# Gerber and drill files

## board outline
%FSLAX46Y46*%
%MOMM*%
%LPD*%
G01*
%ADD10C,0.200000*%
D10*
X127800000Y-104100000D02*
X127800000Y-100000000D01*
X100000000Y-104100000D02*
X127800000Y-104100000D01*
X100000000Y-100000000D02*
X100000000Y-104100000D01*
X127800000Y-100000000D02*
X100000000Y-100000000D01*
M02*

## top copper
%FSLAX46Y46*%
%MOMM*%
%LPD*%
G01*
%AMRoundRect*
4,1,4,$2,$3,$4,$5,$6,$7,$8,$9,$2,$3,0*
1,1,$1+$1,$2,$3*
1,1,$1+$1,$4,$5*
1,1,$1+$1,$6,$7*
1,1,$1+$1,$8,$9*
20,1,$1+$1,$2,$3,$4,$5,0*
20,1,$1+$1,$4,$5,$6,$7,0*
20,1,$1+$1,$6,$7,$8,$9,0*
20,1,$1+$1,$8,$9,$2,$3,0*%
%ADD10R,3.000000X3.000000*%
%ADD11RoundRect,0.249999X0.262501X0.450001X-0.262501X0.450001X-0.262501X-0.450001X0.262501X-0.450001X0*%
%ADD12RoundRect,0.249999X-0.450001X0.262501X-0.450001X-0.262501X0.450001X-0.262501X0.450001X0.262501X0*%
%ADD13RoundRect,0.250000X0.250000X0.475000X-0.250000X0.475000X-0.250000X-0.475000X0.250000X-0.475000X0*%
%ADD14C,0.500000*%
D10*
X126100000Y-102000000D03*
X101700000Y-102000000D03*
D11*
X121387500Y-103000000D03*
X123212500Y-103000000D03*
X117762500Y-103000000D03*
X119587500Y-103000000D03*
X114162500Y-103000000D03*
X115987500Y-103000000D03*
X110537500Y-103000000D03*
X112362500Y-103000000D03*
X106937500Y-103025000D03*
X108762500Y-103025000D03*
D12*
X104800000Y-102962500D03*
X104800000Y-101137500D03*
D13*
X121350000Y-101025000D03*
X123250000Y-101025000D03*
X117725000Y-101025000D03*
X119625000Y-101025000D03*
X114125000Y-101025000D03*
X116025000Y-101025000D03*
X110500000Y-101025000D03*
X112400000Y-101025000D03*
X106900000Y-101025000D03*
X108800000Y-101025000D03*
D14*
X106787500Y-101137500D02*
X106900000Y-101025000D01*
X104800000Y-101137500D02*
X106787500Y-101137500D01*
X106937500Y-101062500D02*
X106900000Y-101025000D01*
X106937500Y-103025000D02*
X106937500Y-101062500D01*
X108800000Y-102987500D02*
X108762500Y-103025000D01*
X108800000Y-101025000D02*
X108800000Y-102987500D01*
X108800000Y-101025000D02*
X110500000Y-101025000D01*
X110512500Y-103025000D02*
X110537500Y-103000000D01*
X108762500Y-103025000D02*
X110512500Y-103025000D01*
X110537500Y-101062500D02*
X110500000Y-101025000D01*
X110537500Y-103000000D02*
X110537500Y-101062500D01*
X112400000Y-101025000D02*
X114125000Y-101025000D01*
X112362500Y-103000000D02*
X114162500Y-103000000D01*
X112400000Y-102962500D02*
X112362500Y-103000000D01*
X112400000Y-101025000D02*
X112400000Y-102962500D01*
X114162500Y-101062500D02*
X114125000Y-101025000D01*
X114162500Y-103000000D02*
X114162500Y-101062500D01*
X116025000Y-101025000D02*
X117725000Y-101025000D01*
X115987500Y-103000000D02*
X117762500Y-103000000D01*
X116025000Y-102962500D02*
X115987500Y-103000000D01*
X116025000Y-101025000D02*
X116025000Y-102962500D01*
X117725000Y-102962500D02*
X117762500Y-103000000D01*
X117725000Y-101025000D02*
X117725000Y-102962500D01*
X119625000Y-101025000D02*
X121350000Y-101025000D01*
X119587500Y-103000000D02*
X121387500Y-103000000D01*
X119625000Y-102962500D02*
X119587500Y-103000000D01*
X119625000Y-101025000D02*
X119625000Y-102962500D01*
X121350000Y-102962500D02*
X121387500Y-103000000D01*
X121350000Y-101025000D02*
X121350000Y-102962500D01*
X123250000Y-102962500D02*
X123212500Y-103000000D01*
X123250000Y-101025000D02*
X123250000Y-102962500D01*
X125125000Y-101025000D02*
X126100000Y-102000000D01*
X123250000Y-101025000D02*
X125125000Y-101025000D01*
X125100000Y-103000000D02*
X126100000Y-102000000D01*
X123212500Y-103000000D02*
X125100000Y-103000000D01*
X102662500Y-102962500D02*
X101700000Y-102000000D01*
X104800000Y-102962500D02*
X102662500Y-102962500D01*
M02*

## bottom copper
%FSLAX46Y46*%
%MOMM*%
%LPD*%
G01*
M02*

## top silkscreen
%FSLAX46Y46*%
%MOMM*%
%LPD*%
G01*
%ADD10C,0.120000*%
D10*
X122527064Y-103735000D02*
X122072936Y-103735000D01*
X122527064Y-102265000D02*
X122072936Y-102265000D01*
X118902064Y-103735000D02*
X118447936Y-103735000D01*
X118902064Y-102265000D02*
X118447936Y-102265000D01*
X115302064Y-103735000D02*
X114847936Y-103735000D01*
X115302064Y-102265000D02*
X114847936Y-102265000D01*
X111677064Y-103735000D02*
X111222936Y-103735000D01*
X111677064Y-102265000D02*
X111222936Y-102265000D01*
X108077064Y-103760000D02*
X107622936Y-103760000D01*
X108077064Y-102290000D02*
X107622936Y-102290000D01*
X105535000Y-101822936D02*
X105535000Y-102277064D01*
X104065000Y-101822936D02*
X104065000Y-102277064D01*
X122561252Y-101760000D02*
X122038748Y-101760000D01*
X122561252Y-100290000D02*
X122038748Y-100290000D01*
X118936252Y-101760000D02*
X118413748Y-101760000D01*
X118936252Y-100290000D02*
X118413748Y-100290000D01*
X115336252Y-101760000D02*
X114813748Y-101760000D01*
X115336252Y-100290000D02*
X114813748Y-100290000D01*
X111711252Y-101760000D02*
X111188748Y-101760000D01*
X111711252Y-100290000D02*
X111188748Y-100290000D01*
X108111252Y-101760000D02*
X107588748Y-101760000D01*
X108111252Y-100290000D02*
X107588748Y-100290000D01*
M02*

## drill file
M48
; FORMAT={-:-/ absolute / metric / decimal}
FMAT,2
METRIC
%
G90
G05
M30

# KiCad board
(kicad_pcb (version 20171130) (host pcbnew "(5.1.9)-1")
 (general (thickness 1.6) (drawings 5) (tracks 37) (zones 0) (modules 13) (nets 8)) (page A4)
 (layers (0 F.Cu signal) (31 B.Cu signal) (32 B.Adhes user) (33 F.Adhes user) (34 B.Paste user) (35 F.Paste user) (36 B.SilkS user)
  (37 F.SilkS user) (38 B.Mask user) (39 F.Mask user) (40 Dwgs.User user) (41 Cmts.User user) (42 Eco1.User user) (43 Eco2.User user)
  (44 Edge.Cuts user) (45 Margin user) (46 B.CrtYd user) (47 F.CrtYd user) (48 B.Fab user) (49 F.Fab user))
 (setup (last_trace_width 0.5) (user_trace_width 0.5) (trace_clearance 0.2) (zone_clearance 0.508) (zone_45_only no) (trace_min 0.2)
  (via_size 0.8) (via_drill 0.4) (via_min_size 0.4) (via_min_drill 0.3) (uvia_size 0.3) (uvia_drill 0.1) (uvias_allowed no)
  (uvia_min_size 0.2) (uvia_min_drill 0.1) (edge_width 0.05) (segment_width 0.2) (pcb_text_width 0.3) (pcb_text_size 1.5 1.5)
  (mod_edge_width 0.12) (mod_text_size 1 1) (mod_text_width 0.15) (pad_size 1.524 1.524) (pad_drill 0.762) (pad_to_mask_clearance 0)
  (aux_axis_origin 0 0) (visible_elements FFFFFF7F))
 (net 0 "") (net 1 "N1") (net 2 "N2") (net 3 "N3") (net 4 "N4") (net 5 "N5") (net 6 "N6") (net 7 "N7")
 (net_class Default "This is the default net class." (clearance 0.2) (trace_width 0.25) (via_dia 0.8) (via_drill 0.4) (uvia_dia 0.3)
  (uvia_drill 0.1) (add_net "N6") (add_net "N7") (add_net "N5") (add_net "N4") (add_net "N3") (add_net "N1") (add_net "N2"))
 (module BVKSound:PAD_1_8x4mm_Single (layer F.Cu) (at 126.1 102)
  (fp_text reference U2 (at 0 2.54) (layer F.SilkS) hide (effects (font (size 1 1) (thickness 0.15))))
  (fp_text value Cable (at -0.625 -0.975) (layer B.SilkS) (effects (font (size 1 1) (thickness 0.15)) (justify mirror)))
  (pad 1 smd rect (at 0 0) (size 3 3) (layers F.Cu F.Paste F.Mask) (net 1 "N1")))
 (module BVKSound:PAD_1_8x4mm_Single (layer F.Cu) (at 102.025 102)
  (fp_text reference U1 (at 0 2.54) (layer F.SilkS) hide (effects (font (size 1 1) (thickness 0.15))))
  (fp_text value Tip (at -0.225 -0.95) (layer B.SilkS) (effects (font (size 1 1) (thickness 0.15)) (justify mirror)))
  (pad 1 smd rect (at -0.325 0) (size 3 3) (layers F.Cu F.Paste F.Mask) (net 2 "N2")))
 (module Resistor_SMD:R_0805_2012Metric (layer F.Cu) (at 122.3 103 180)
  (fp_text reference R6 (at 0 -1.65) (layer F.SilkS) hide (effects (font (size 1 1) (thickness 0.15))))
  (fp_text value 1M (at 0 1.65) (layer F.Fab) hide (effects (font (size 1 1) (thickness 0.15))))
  (fp_line (start -0.227064 -0.735) (end 0.227064 -0.735) (layer F.SilkS) (width 0.12))
  (fp_line (start -0.227064 0.735) (end 0.227064 0.735) (layer F.SilkS) (width 0.12))
  (pad 2 smd roundrect (at 0.9125 0 180) (size 1.025 1.4) (layers F.Cu F.Paste F.Mask) (roundrect_rratio 0.2439014634146341) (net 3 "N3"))
  (pad 1 smd roundrect (at -0.9125 0 180) (size 1.025 1.4) (layers F.Cu F.Paste F.Mask) (roundrect_rratio 0.2439014634146341) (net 1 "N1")))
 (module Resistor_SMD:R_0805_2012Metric (layer F.Cu) (at 118.675 103 180)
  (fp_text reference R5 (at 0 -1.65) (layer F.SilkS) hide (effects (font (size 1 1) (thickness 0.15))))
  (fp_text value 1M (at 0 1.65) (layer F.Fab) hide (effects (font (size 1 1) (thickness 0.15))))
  (fp_line (start -0.227064 -0.735) (end 0.227064 -0.735) (layer F.SilkS) (width 0.12))
  (fp_line (start -0.227064 0.735) (end 0.227064 0.735) (layer F.SilkS) (width 0.12))
  (pad 2 smd roundrect (at 0.9125 0 180) (size 1.025 1.4) (layers F.Cu F.Paste F.Mask) (roundrect_rratio 0.2439014634146341) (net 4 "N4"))
  (pad 1 smd roundrect (at -0.9125 0 180) (size 1.025 1.4) (layers F.Cu F.Paste F.Mask) (roundrect_rratio 0.2439014634146341) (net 3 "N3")))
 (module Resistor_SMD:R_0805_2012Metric (layer F.Cu) (at 115.075 103 180)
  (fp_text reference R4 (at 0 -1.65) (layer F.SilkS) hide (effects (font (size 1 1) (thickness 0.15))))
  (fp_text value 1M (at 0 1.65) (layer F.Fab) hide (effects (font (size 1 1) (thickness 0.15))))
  (fp_line (start -0.227064 -0.735) (end 0.227064 -0.735) (layer F.SilkS) (width 0.12))
  (fp_line (start -0.227064 0.735) (end 0.227064 0.735) (layer F.SilkS) (width 0.12))
  (pad 2 smd roundrect (at 0.9125 0 180) (size 1.025 1.4) (layers F.Cu F.Paste F.Mask) (roundrect_rratio 0.2439014634146341) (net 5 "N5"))
  (pad 1 smd roundrect (at -0.9125 0 180) (size 1.025 1.4) (layers F.Cu F.Paste F.Mask) (roundrect_rratio 0.2439014634146341) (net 4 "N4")))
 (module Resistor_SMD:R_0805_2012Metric (layer F.Cu) (at 111.45 103 180)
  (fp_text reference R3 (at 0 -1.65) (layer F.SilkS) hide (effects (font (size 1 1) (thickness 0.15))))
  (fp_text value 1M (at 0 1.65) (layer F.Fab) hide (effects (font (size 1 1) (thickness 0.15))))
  (fp_line (start -0.227064 -0.735) (end 0.227064 -0.735) (layer F.SilkS) (width 0.12))
  (fp_line (start -0.227064 0.735) (end 0.227064 0.735) (layer F.SilkS) (width 0.12))
  (pad 2 smd roundrect (at 0.9125 0 180) (size 1.025 1.4) (layers F.Cu F.Paste F.Mask) (roundrect_rratio 0.2439014634146341) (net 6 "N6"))
  (pad 1 smd roundrect (at -0.9125 0 180) (size 1.025 1.4) (layers F.Cu F.Paste F.Mask) (roundrect_rratio 0.2439014634146341) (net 5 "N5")))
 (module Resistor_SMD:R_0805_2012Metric (layer F.Cu) (at 107.85 103.025 180)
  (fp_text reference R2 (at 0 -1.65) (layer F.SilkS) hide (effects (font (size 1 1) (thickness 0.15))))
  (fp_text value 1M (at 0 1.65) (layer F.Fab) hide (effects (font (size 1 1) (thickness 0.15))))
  (fp_line (start -0.227064 -0.735) (end 0.227064 -0.735) (layer F.SilkS) (width 0.12))
  (fp_line (start -0.227064 0.735) (end 0.227064 0.735) (layer F.SilkS) (width 0.12))
  (pad 2 smd roundrect (at 0.9125 0 180) (size 1.025 1.4) (layers F.Cu F.Paste F.Mask) (roundrect_rratio 0.2439014634146341) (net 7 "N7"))
  (pad 1 smd roundrect (at -0.9125 0 180) (size 1.025 1.4) (layers F.Cu F.Paste F.Mask) (roundrect_rratio 0.2439014634146341) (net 6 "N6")))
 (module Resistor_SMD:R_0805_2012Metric (layer F.Cu) (at 104.8 102.05 270)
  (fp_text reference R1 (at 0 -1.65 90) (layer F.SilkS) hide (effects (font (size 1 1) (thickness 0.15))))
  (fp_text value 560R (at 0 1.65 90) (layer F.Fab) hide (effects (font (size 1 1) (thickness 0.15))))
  (fp_line (start -0.227064 -0.735) (end 0.227064 -0.735) (layer F.SilkS) (width 0.12))
  (fp_line (start -0.227064 0.735) (end 0.227064 0.735) (layer F.SilkS) (width 0.12))
  (pad 2 smd roundrect (at 0.9125 0 270) (size 1.025 1.4) (layers F.Cu F.Paste F.Mask) (roundrect_rratio 0.2439014634146341) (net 2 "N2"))
  (pad 1 smd roundrect (at -0.9125 0 270) (size 1.025 1.4) (layers F.Cu F.Paste F.Mask) (roundrect_rratio 0.2439014634146341) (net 7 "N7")))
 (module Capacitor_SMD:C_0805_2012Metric (layer F.Cu) (at 122.3 101.025 180)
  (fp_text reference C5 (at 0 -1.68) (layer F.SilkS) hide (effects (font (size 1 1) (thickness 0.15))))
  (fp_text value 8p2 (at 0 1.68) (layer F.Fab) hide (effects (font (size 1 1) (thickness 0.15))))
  (fp_line (start -0.261252 -0.735) (end 0.261252 -0.735) (layer F.SilkS) (width 0.12))
  (fp_line (start -0.261252 0.735) (end 0.261252 0.735) (layer F.SilkS) (width 0.12))
  (pad 2 smd roundrect (at 0.95 0 180) (size 1 1.45) (layers F.Cu F.Paste F.Mask) (roundrect_rratio 0.25) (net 3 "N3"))
  (pad 1 smd roundrect (at -0.95 0 180) (size 1 1.45) (layers F.Cu F.Paste F.Mask) (roundrect_rratio 0.25) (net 1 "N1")))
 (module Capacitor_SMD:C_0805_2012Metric (layer F.Cu) (at 118.675 101.025 180)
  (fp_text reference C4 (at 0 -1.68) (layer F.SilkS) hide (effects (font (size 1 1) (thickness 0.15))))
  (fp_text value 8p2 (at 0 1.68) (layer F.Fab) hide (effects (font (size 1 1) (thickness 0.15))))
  (fp_line (start -0.261252 -0.735) (end 0.261252 -0.735) (layer F.SilkS) (width 0.12))
  (fp_line (start -0.261252 0.735) (end 0.261252 0.735) (layer F.SilkS) (width 0.12))
  (pad 2 smd roundrect (at 0.95 0 180) (size 1 1.45) (layers F.Cu F.Paste F.Mask) (roundrect_rratio 0.25) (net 4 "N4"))
  (pad 1 smd roundrect (at -0.95 0 180) (size 1 1.45) (layers F.Cu F.Paste F.Mask) (roundrect_rratio 0.25) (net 3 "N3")))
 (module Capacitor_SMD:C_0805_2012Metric (layer F.Cu) (at 115.075 101.025 180)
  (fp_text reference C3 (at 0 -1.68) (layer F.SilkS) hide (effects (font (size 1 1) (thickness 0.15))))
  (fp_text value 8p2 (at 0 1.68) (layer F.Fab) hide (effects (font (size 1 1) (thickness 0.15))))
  (fp_line (start -0.261252 -0.735) (end 0.261252 -0.735) (layer F.SilkS) (width 0.12))
  (fp_line (start -0.261252 0.735) (end 0.261252 0.735) (layer F.SilkS) (width 0.12))
  (pad 2 smd roundrect (at 0.95 0 180) (size 1 1.45) (layers F.Cu F.Paste F.Mask) (roundrect_rratio 0.25) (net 5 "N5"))
  (pad 1 smd roundrect (at -0.95 0 180) (size 1 1.45) (layers F.Cu F.Paste F.Mask) (roundrect_rratio 0.25) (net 4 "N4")))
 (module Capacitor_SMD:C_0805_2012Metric (layer F.Cu) (at 111.45 101.025 180)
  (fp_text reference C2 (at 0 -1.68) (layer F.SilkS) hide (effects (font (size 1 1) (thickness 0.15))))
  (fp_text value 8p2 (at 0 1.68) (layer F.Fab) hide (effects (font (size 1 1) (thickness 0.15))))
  (fp_line (start -0.261252 -0.735) (end 0.261252 -0.735) (layer F.SilkS) (width 0.12))
  (fp_line (start -0.261252 0.735) (end 0.261252 0.735) (layer F.SilkS) (width 0.12))
  (pad 2 smd roundrect (at 0.95 0 180) (size 1 1.45) (layers F.Cu F.Paste F.Mask) (roundrect_rratio 0.25) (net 6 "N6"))
  (pad 1 smd roundrect (at -0.95 0 180) (size 1 1.45) (layers F.Cu F.Paste F.Mask) (roundrect_rratio 0.25) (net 5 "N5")))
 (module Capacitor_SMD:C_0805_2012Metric (layer F.Cu) (at 107.85 101.025 180)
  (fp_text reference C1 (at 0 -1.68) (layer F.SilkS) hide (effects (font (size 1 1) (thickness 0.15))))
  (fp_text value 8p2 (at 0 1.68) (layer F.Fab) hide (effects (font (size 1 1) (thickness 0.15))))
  (fp_line (start -0.261252 -0.735) (end 0.261252 -0.735) (layer F.SilkS) (width 0.12))
  (fp_line (start -0.261252 0.735) (end 0.261252 0.735) (layer F.SilkS) (width 0.12))
  (pad 2 smd roundrect (at 0.95 0 180) (size 1 1.45) (layers F.Cu F.Paste F.Mask) (roundrect_rratio 0.25) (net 7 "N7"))
  (pad 1 smd roundrect (at -0.95 0 180) (size 1 1.45) (layers F.Cu F.Paste F.Mask) (roundrect_rratio 0.25) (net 6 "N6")))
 (gr_line (start 127.8 104.1) (end 127.8 100) (layer Edge.Cuts) (width 0.2))
 (gr_line (start 100 104.1) (end 127.8 104.1) (layer Edge.Cuts) (width 0.2))
 (gr_line (start 100 100) (end 100 104.1) (layer Edge.Cuts) (width 0.2))
 (gr_line (start 127.8 100) (end 100 100) (layer Edge.Cuts) (width 0.2))
 (segment (start 106.7875 101.1375) (end 106.9 101.025) (width 0.5) (layer F.Cu) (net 7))
 (segment (start 104.8 101.1375) (end 106.7875 101.1375) (width 0.5) (layer F.Cu) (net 7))
 (segment (start 106.9375 101.0625) (end 106.9 101.025) (width 0.5) (layer F.Cu) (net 7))
 (segment (start 106.9375 103.025) (end 106.9375 101.0625) (width 0.5) (layer F.Cu) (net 7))
 (segment (start 108.8 102.9875) (end 108.7625 103.025) (width 0.5) (layer F.Cu) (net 6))
 (segment (start 108.8 101.025) (end 108.8 102.9875) (width 0.5) (layer F.Cu) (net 6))
 (segment (start 108.8 101.025) (end 110.5 101.025) (width 0.5) (layer F.Cu) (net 6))
 (segment (start 110.5125 103.025) (end 110.5375 103) (width 0.5) (layer F.Cu) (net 6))
 (segment (start 108.7625 103.025) (end 110.5125 103.025) (width 0.5) (layer F.Cu) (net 6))
 (segment (start 110.5375 101.0625) (end 110.5 101.025) (width 0.5) (layer F.Cu) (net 6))
 (segment (start 110.5375 103) (end 110.5375 101.0625) (width 0.5) (layer F.Cu) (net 6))
 (segment (start 112.4 101.025) (end 114.125 101.025) (width 0.5) (layer F.Cu) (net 5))
 (segment (start 112.3625 103) (end 114.1625 103) (width 0.5) (layer F.Cu) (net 5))
 (segment (start 112.4 102.9625) (end 112.3625 103) (width 0.5) (layer F.Cu) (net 5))
 (segment (start 112.4 101.025) (end 112.4 102.9625) (width 0.5) (layer F.Cu) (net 5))
 (segment (start 114.1625 101.0625) (end 114.125 101.025) (width 0.5) (layer F.Cu) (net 5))
 (segment (start 114.1625 103) (end 114.1625 101.0625) (width 0.5) (layer F.Cu) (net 5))
 (segment (start 116.025 101.025) (end 117.725 101.025) (width 0.5) (layer F.Cu) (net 4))
 (segment (start 115.9875 103) (end 117.7625 103) (width 0.5) (layer F.Cu) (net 4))
 (segment (start 116.025 102.9625) (end 115.9875 103) (width 0.5) (layer F.Cu) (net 4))
 (segment (start 116.025 101.025) (end 116.025 102.9625) (width 0.5) (layer F.Cu) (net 4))
 (segment (start 117.725 102.9625) (end 117.7625 103) (width 0.5) (layer F.Cu) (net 4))
 (segment (start 117.725 101.025) (end 117.725 102.9625) (width 0.5) (layer F.Cu) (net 4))
 (segment (start 119.625 101.025) (end 121.35 101.025) (width 0.5) (layer F.Cu) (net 3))
 (segment (start 119.5875 103) (end 121.3875 103) (width 0.5) (layer F.Cu) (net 3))
 (segment (start 119.625 102.9625) (end 119.5875 103) (width 0.5) (layer F.Cu) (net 3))
 (segment (start 119.625 101.025) (end 119.625 102.9625) (width 0.5) (layer F.Cu) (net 3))
 (segment (start 121.35 102.9625) (end 121.3875 103) (width 0.5) (layer F.Cu) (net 3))
 (segment (start 121.35 101.025) (end 121.35 102.9625) (width 0.5) (layer F.Cu) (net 3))
 (segment (start 123.25 102.9625) (end 123.2125 103) (width 0.5) (layer F.Cu) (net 1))
 (segment (start 123.25 101.025) (end 123.25 102.9625) (width 0.5) (layer F.Cu) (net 1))
 (segment (start 125.125 101.025) (end 126.1 102) (width 0.5) (layer F.Cu) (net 1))
 (segment (start 123.25 101.025) (end 125.125 101.025) (width 0.5) (layer F.Cu) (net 1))
 (segment (start 125.1 103) (end 126.1 102) (width 0.5) (layer F.Cu) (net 1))
 (segment (start 123.2125 103) (end 125.1 103) (width 0.5) (layer F.Cu) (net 1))
 (segment (start 102.6625 102.9625) (end 101.7 102) (width 0.5) (layer F.Cu) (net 2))
 (segment (start 104.8 102.9625) (end 102.6625 102.9625) (width 0.5) (layer F.Cu) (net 2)))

